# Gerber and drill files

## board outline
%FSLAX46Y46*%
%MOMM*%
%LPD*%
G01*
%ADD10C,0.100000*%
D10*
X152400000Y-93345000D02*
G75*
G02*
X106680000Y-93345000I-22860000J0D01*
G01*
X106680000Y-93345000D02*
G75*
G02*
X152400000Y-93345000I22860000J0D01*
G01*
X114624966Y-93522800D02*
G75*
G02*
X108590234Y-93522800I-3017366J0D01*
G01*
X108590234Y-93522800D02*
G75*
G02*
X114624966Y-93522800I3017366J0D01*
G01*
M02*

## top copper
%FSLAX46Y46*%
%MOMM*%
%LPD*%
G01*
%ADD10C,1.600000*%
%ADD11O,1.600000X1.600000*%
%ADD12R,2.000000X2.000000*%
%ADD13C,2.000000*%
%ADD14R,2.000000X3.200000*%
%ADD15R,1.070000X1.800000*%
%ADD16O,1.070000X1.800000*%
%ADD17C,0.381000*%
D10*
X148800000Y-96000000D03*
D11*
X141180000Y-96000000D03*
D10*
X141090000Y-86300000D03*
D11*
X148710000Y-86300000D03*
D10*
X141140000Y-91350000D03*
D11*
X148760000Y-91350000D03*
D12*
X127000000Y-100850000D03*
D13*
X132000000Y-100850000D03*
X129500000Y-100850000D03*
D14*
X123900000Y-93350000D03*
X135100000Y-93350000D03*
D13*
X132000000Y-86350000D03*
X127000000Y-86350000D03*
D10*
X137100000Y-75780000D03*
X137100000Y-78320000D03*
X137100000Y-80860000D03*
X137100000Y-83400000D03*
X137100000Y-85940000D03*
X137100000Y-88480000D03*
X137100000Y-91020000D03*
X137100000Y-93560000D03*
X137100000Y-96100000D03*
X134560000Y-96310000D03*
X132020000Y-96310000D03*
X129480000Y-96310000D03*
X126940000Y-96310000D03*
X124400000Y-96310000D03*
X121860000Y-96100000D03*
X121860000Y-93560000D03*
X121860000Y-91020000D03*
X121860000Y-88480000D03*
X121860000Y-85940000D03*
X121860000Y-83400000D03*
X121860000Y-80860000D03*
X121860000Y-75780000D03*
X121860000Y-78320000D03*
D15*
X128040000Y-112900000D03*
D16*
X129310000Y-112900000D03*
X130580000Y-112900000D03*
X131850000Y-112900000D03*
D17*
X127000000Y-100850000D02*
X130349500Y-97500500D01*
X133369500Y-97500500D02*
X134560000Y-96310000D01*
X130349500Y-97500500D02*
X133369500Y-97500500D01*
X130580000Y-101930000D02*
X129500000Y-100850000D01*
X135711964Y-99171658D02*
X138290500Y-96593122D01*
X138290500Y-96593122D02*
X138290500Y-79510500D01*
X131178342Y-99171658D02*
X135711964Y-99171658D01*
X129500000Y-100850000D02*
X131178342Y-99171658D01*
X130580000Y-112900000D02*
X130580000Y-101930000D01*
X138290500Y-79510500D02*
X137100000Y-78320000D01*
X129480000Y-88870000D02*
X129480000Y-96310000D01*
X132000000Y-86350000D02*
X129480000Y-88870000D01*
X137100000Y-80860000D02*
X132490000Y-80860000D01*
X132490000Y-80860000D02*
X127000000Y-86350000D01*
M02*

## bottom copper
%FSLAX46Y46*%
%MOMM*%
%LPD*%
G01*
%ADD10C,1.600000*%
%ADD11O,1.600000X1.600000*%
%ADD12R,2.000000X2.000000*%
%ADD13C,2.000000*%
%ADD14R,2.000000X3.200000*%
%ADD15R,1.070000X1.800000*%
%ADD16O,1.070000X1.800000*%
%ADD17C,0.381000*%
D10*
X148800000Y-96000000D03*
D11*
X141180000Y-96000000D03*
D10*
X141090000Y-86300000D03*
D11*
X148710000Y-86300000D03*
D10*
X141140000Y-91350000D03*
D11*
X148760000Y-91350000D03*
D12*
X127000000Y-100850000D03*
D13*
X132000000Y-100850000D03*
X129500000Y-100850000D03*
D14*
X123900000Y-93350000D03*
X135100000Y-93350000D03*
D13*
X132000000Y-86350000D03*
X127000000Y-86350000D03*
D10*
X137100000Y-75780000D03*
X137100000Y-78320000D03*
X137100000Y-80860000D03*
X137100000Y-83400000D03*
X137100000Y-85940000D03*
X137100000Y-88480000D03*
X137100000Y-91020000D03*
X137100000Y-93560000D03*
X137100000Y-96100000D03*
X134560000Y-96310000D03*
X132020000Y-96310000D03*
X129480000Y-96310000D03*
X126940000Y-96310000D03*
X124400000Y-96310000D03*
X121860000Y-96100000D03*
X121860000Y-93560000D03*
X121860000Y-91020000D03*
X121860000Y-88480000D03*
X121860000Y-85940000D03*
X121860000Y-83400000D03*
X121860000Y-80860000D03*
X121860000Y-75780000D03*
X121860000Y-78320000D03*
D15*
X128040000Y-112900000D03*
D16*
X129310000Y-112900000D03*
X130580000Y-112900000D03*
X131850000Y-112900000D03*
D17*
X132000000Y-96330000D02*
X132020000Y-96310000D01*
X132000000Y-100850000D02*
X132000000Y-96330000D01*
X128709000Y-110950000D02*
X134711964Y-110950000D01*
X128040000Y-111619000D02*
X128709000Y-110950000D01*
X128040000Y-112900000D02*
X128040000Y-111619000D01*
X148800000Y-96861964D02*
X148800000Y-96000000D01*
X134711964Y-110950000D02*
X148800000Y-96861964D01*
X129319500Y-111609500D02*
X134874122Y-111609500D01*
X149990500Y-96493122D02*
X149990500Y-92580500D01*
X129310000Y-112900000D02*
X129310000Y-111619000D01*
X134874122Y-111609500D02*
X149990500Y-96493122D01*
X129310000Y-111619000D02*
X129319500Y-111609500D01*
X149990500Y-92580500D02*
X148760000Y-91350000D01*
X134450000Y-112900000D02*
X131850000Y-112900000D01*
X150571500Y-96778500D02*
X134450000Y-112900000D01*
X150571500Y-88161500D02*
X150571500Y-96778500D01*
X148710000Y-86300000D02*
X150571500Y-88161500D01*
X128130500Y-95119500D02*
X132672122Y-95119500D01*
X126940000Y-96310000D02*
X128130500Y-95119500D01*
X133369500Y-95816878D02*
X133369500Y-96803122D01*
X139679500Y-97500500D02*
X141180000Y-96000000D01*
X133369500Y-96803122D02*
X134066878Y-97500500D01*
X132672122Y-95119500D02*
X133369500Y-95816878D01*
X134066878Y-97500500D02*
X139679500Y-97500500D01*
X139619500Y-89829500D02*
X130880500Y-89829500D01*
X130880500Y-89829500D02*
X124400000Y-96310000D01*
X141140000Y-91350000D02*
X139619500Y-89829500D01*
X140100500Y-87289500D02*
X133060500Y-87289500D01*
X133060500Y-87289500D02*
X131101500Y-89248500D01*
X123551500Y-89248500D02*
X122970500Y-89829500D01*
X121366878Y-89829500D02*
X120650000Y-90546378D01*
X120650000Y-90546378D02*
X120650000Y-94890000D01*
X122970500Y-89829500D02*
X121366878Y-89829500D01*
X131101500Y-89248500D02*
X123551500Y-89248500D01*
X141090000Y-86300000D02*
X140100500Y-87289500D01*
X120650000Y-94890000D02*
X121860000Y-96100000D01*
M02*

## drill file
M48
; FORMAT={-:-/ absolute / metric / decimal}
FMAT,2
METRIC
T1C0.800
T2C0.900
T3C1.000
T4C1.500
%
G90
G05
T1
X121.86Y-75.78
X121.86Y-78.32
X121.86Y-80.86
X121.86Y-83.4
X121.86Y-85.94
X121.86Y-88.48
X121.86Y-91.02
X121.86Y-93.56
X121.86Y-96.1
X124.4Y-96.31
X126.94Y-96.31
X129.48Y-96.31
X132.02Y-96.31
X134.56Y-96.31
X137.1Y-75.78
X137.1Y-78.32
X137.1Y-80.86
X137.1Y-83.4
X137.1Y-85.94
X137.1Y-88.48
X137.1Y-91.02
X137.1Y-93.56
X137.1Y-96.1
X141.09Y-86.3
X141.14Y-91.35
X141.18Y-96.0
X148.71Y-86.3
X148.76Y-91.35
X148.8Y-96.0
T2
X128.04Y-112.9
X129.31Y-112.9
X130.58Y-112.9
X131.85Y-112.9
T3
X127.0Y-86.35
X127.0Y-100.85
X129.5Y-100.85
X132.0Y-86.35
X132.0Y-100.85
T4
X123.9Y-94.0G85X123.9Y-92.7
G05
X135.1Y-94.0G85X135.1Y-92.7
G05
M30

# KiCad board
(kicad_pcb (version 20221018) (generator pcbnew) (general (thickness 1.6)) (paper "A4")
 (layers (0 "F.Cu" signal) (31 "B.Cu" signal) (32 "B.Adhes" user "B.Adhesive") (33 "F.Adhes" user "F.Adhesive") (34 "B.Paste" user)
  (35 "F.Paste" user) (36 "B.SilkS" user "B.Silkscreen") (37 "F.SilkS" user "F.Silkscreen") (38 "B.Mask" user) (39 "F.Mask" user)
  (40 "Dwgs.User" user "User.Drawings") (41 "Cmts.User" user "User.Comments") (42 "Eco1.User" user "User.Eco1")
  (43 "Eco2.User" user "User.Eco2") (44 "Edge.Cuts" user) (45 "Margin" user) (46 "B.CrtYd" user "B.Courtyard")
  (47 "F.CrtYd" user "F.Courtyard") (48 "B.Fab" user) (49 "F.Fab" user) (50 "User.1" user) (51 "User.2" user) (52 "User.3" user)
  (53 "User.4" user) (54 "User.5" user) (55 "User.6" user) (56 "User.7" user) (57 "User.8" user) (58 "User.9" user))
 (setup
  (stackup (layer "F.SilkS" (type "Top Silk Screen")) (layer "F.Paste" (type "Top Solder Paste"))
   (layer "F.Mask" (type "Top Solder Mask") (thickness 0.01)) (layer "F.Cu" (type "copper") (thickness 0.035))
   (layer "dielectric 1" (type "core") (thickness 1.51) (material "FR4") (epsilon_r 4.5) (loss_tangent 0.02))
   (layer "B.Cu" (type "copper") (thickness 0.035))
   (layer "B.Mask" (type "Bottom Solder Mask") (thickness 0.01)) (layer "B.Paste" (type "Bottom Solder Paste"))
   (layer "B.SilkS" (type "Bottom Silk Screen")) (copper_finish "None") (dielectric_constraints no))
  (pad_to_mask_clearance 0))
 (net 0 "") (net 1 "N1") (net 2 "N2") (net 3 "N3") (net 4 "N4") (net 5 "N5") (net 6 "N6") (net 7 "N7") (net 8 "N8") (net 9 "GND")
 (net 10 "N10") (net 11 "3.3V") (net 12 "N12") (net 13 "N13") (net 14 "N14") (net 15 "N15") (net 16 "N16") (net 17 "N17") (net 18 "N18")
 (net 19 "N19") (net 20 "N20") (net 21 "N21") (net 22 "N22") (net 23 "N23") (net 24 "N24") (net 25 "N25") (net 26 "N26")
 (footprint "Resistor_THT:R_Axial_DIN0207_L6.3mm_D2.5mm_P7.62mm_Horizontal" (layer "F.Cu") (at 148.8 96 180)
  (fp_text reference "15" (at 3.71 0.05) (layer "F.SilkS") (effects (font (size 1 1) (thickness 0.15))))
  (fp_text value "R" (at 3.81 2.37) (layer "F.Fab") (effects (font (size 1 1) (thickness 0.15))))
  (pad "1" thru_hole circle (at 0 0 180) (size 1.6 1.6) (drill 0.8) (layers "*.Cu" "*.Mask") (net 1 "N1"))
  (pad "2" thru_hole oval (at 7.62 0 180) (size 1.6 1.6) (drill 0.8) (layers "*.Cu" "*.Mask") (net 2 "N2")))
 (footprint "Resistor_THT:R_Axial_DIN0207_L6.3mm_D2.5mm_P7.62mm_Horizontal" (layer "F.Cu") (at 141.09 86.3)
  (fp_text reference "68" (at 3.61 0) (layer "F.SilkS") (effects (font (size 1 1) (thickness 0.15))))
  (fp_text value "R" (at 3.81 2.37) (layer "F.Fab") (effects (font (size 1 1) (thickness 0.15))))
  (pad "1" thru_hole circle (at 0 0) (size 1.6 1.6) (drill 0.8) (layers "*.Cu" "*.Mask") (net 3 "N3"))
  (pad "2" thru_hole oval (at 7.62 0) (size 1.6 1.6) (drill 0.8) (layers "*.Cu" "*.Mask") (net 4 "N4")))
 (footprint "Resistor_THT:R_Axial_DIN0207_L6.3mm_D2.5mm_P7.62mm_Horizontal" (layer "F.Cu") (at 141.14 91.35)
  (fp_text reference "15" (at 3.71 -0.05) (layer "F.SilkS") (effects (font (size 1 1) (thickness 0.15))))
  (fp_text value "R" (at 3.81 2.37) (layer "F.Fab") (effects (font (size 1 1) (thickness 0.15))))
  (pad "1" thru_hole circle (at 0 0) (size 1.6 1.6) (drill 0.8) (layers "*.Cu" "*.Mask") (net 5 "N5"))
  (pad "2" thru_hole oval (at 7.62 0) (size 1.6 1.6) (drill 0.8) (layers "*.Cu" "*.Mask") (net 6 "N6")))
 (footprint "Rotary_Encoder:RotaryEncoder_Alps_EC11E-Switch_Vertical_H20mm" (layer "F.Cu") (at 127 100.85 90)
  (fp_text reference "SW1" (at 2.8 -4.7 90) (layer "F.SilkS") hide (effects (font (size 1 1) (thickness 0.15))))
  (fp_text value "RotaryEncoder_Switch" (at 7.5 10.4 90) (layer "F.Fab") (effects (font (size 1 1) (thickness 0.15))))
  (pad "A" thru_hole rect (at 0 0 90) (size 2 2) (drill 1) (layers "*.Cu" "*.Mask") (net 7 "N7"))
  (pad "B" thru_hole circle (at 0 5 90) (size 2 2) (drill 1) (layers "*.Cu" "*.Mask") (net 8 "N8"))
  (pad "C" thru_hole circle (at 0 2.5 90) (size 2 2) (drill 1) (layers "*.Cu" "*.Mask") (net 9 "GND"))
  (pad "MP" thru_hole rect (at 7.5 -3.1 90) (size 3.2 2) (drill oval 2.8 1.5) (layers "*.Cu" "*.Mask"))
  (pad "MP" thru_hole rect (at 7.5 8.1 90) (size 3.2 2) (drill oval 2.8 1.5) (layers "*.Cu" "*.Mask"))
  (pad "S1" thru_hole circle (at 14.5 5 90) (size 2 2) (drill 1) (layers "*.Cu" "*.Mask") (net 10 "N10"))
  (pad "S2" thru_hole circle (at 14.5 0 90) (size 2 2) (drill 1) (layers "*.Cu" "*.Mask") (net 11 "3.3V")))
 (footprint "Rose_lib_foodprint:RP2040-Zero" (layer "F.Cu") (at 120.48 97.69)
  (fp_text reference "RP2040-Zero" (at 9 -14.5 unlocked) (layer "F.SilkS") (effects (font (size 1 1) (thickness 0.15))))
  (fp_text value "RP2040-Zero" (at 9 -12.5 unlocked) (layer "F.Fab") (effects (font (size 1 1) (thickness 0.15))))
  (pad "1" thru_hole circle (at 16.62 -21.91) (size 1.6 1.6) (drill 0.8) (layers "*.Cu" "*.Mask") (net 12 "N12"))
  (pad "2" thru_hole circle (at 16.62 -19.37) (size 1.6 1.6) (drill 0.8) (layers "*.Cu" "*.Mask") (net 9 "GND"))
  (pad "3" thru_hole circle (at 16.62 -16.83) (size 1.6 1.6) (drill 0.8) (layers "*.Cu" "*.Mask") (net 11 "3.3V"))
  (pad "4" thru_hole circle (at 16.62 -14.29) (size 1.6 1.6) (drill 0.8) (layers "*.Cu" "*.Mask") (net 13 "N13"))
  (pad "5" thru_hole circle (at 16.62 -11.75) (size 1.6 1.6) (drill 0.8) (layers "*.Cu" "*.Mask") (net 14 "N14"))
  (pad "6" thru_hole circle (at 16.62 -9.21) (size 1.6 1.6) (drill 0.8) (layers "*.Cu" "*.Mask") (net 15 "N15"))
  (pad "7" thru_hole circle (at 16.62 -6.67) (size 1.6 1.6) (drill 0.8) (layers "*.Cu" "*.Mask") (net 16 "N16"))
  (pad "8" thru_hole circle (at 16.62 -4.13) (size 1.6 1.6) (drill 0.8) (layers "*.Cu" "*.Mask") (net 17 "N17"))
  (pad "9" thru_hole circle (at 16.62 -1.59) (size 1.6 1.6) (drill 0.8) (layers "*.Cu" "*.Mask") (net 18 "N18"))
  (pad "10" thru_hole circle (at 14.08 -1.38) (size 1.6 1.6) (drill 0.8) (layers "*.Cu" "*.Mask") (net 7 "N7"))
  (pad "11" thru_hole circle (at 11.54 -1.38) (size 1.6 1.6) (drill 0.8) (layers "*.Cu" "*.Mask") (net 8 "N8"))
  (pad "12" thru_hole circle (at 9 -1.38) (size 1.6 1.6) (drill 0.8) (layers "*.Cu" "*.Mask") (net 10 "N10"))
  (pad "13" thru_hole circle (at 6.46 -1.38) (size 1.6 1.6) (drill 0.8) (layers "*.Cu" "*.Mask") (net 2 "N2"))
  (pad "14" thru_hole circle (at 3.92 -1.38) (size 1.6 1.6) (drill 0.8) (layers "*.Cu" "*.Mask") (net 5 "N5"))
  (pad "15" thru_hole circle (at 1.38 -1.59) (size 1.6 1.6) (drill 0.8) (layers "*.Cu" "*.Mask") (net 3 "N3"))
  (pad "16" thru_hole circle (at 1.38 -4.13) (size 1.6 1.6) (drill 0.8) (layers "*.Cu" "*.Mask") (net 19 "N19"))
  (pad "17" thru_hole circle (at 1.38 -6.67) (size 1.6 1.6) (drill 0.8) (layers "*.Cu" "*.Mask") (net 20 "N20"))
  (pad "18" thru_hole circle (at 1.38 -9.21) (size 1.6 1.6) (drill 0.8) (layers "*.Cu" "*.Mask") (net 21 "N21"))
  (pad "19" thru_hole circle (at 1.38 -11.75) (size 1.6 1.6) (drill 0.8) (layers "*.Cu" "*.Mask") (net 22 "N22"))
  (pad "20" thru_hole circle (at 1.38 -14.29) (size 1.6 1.6) (drill 0.8) (layers "*.Cu" "*.Mask") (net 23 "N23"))
  (pad "21" thru_hole circle (at 1.38 -16.83) (size 1.6 1.6) (drill 0.8) (layers "*.Cu" "*.Mask") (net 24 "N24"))
  (pad "22" thru_hole circle (at 1.38 -21.91) (size 1.6 1.6) (drill 0.8) (layers "*.Cu" "*.Mask") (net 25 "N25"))
  (pad "23" thru_hole circle (at 1.38 -19.37) (size 1.6 1.6) (drill 0.8) (layers "*.Cu" "*.Mask") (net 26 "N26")))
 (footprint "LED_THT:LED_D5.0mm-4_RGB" (layer "F.Cu") (at 128.04 112.9)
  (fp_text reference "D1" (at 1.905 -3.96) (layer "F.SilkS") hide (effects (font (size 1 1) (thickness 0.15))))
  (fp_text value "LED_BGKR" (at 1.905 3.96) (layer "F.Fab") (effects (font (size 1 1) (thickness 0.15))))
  (pad "1" thru_hole rect (at 0 0) (size 1.07 1.8) (drill 0.9) (layers "*.Cu" "*.Mask") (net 1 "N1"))
  (pad "2" thru_hole oval (at 1.27 0) (size 1.07 1.8) (drill 0.9) (layers "*.Cu" "*.Mask") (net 6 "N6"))
  (pad "3" thru_hole oval (at 2.54 0) (size 1.07 1.8) (drill 0.9) (layers "*.Cu" "*.Mask") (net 9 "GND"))
  (pad "4" thru_hole oval (at 3.81 0) (size 1.07 1.8) (drill 0.9) (layers "*.Cu" "*.Mask") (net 4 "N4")))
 (gr_circle (center 129.54 93.345) (end 129.54 70.485) (stroke (width 0.1) (type default)) (fill none) (layer "Edge.Cuts"))
 (gr_circle (center 111.6076 93.5228) (end 113.7412 91.3892) (stroke (width 0.1) (type default)) (fill none) (layer "Edge.Cuts"))
 (segment (start 127 100.85) (end 130.3495 97.5005) (width 0.381) (layer "F.Cu") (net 7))
 (segment (start 133.3695 97.5005) (end 134.56 96.31) (width 0.381) (layer "F.Cu") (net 7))
 (segment (start 130.3495 97.5005) (end 133.3695 97.5005) (width 0.381) (layer "F.Cu") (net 7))
 (segment (start 132 96.33) (end 132.02 96.31) (width 0.381) (layer "B.Cu") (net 8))
 (segment (start 132 100.85) (end 132 96.33) (width 0.381) (layer "B.Cu") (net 8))
 (segment (start 130.58 101.93) (end 129.5 100.85) (width 0.381) (layer "F.Cu") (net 9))
 (segment (start 135.711964 99.171658) (end 138.2905 96.593122) (width 0.381) (layer "F.Cu") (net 9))
 (segment (start 138.2905 96.593122) (end 138.2905 79.5105) (width 0.381) (layer "F.Cu") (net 9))
 (segment (start 131.178342 99.171658) (end 135.711964 99.171658) (width 0.381) (layer "F.Cu") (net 9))
 (segment (start 129.5 100.85) (end 131.178342 99.171658) (width 0.381) (layer "F.Cu") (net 9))
 (segment (start 130.58 112.9) (end 130.58 101.93) (width 0.381) (layer "F.Cu") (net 9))
 (segment (start 138.2905 79.5105) (end 137.1 78.32) (width 0.381) (layer "F.Cu") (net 9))
 (segment (start 129.48 88.87) (end 129.48 96.31) (width 0.381) (layer "F.Cu") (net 10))
 (segment (start 132 86.35) (end 129.48 88.87) (width 0.381) (layer "F.Cu") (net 10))
 (segment (start 137.1 80.86) (end 132.49 80.86) (width 0.381) (layer "F.Cu") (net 11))
 (segment (start 132.49 80.86) (end 127 86.35) (width 0.381) (layer "F.Cu") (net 11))
 (segment (start 128.709 110.95) (end 134.711964 110.95) (width 0.381) (layer "B.Cu") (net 1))
 (segment (start 128.04 111.619) (end 128.709 110.95) (width 0.381) (layer "B.Cu") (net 1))
 (segment (start 128.04 112.9) (end 128.04 111.619) (width 0.381) (layer "B.Cu") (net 1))
 (segment (start 148.8 96.861964) (end 148.8 96) (width 0.381) (layer "B.Cu") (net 1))
 (segment (start 134.711964 110.95) (end 148.8 96.861964) (width 0.381) (layer "B.Cu") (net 1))
 (segment (start 129.3195 111.6095) (end 134.874122 111.6095) (width 0.381) (layer "B.Cu") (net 6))
 (segment (start 149.9905 96.493122) (end 149.9905 92.5805) (width 0.381) (layer "B.Cu") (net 6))
 (segment (start 129.31 112.9) (end 129.31 111.619) (width 0.381) (layer "B.Cu") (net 6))
 (segment (start 134.874122 111.6095) (end 149.9905 96.493122) (width 0.381) (layer "B.Cu") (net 6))
 (segment (start 129.31 111.619) (end 129.3195 111.6095) (width 0.381) (layer "B.Cu") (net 6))
 (segment (start 149.9905 92.5805) (end 148.76 91.35) (width 0.381) (layer "B.Cu") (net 6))
 (segment (start 134.45 112.9) (end 131.85 112.9) (width 0.381) (layer "B.Cu") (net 4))
 (segment (start 150.5715 96.7785) (end 134.45 112.9) (width 0.381) (layer "B.Cu") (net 4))
 (segment (start 150.5715 88.1615) (end 150.5715 96.7785) (width 0.381) (layer "B.Cu") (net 4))
 (segment (start 148.71 86.3) (end 150.5715 88.1615) (width 0.381) (layer "B.Cu") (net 4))
 (segment (start 128.1305 95.1195) (end 132.672122 95.1195) (width 0.381) (layer "B.Cu") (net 2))
 (segment (start 126.94 96.31) (end 128.1305 95.1195) (width 0.381) (layer "B.Cu") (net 2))
 (segment (start 133.3695 95.816878) (end 133.3695 96.803122) (width 0.381) (layer "B.Cu") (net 2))
 (segment (start 139.6795 97.5005) (end 141.18 96) (width 0.381) (layer "B.Cu") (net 2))
 (segment (start 133.3695 96.803122) (end 134.066878 97.5005) (width 0.381) (layer "B.Cu") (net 2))
 (segment (start 132.672122 95.1195) (end 133.3695 95.816878) (width 0.381) (layer "B.Cu") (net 2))
 (segment (start 134.066878 97.5005) (end 139.6795 97.5005) (width 0.381) (layer "B.Cu") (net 2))
 (segment (start 139.6195 89.8295) (end 130.8805 89.8295) (width 0.381) (layer "B.Cu") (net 5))
 (segment (start 130.8805 89.8295) (end 124.4 96.31) (width 0.381) (layer "B.Cu") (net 5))
 (segment (start 141.14 91.35) (end 139.6195 89.8295) (width 0.381) (layer "B.Cu") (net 5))
 (segment (start 140.1005 87.2895) (end 133.0605 87.2895) (width 0.381) (layer "B.Cu") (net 3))
 (segment (start 133.0605 87.2895) (end 131.1015 89.2485) (width 0.381) (layer "B.Cu") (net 3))
 (segment (start 123.5515 89.2485) (end 122.9705 89.8295) (width 0.381) (layer "B.Cu") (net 3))
 (segment (start 121.366878 89.8295) (end 120.65 90.546378) (width 0.381) (layer "B.Cu") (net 3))
 (segment (start 120.65 90.546378) (end 120.65 94.89) (width 0.381) (layer "B.Cu") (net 3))
 (segment (start 122.9705 89.8295) (end 121.366878 89.8295) (width 0.381) (layer "B.Cu") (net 3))
 (segment (start 131.1015 89.2485) (end 123.5515 89.2485) (width 0.381) (layer "B.Cu") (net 3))
 (segment (start 141.09 86.3) (end 140.1005 87.2895) (width 0.381) (layer "B.Cu") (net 3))
 (segment (start 120.65 94.89) (end 121.86 96.1) (width 0.381) (layer "B.Cu") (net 3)))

